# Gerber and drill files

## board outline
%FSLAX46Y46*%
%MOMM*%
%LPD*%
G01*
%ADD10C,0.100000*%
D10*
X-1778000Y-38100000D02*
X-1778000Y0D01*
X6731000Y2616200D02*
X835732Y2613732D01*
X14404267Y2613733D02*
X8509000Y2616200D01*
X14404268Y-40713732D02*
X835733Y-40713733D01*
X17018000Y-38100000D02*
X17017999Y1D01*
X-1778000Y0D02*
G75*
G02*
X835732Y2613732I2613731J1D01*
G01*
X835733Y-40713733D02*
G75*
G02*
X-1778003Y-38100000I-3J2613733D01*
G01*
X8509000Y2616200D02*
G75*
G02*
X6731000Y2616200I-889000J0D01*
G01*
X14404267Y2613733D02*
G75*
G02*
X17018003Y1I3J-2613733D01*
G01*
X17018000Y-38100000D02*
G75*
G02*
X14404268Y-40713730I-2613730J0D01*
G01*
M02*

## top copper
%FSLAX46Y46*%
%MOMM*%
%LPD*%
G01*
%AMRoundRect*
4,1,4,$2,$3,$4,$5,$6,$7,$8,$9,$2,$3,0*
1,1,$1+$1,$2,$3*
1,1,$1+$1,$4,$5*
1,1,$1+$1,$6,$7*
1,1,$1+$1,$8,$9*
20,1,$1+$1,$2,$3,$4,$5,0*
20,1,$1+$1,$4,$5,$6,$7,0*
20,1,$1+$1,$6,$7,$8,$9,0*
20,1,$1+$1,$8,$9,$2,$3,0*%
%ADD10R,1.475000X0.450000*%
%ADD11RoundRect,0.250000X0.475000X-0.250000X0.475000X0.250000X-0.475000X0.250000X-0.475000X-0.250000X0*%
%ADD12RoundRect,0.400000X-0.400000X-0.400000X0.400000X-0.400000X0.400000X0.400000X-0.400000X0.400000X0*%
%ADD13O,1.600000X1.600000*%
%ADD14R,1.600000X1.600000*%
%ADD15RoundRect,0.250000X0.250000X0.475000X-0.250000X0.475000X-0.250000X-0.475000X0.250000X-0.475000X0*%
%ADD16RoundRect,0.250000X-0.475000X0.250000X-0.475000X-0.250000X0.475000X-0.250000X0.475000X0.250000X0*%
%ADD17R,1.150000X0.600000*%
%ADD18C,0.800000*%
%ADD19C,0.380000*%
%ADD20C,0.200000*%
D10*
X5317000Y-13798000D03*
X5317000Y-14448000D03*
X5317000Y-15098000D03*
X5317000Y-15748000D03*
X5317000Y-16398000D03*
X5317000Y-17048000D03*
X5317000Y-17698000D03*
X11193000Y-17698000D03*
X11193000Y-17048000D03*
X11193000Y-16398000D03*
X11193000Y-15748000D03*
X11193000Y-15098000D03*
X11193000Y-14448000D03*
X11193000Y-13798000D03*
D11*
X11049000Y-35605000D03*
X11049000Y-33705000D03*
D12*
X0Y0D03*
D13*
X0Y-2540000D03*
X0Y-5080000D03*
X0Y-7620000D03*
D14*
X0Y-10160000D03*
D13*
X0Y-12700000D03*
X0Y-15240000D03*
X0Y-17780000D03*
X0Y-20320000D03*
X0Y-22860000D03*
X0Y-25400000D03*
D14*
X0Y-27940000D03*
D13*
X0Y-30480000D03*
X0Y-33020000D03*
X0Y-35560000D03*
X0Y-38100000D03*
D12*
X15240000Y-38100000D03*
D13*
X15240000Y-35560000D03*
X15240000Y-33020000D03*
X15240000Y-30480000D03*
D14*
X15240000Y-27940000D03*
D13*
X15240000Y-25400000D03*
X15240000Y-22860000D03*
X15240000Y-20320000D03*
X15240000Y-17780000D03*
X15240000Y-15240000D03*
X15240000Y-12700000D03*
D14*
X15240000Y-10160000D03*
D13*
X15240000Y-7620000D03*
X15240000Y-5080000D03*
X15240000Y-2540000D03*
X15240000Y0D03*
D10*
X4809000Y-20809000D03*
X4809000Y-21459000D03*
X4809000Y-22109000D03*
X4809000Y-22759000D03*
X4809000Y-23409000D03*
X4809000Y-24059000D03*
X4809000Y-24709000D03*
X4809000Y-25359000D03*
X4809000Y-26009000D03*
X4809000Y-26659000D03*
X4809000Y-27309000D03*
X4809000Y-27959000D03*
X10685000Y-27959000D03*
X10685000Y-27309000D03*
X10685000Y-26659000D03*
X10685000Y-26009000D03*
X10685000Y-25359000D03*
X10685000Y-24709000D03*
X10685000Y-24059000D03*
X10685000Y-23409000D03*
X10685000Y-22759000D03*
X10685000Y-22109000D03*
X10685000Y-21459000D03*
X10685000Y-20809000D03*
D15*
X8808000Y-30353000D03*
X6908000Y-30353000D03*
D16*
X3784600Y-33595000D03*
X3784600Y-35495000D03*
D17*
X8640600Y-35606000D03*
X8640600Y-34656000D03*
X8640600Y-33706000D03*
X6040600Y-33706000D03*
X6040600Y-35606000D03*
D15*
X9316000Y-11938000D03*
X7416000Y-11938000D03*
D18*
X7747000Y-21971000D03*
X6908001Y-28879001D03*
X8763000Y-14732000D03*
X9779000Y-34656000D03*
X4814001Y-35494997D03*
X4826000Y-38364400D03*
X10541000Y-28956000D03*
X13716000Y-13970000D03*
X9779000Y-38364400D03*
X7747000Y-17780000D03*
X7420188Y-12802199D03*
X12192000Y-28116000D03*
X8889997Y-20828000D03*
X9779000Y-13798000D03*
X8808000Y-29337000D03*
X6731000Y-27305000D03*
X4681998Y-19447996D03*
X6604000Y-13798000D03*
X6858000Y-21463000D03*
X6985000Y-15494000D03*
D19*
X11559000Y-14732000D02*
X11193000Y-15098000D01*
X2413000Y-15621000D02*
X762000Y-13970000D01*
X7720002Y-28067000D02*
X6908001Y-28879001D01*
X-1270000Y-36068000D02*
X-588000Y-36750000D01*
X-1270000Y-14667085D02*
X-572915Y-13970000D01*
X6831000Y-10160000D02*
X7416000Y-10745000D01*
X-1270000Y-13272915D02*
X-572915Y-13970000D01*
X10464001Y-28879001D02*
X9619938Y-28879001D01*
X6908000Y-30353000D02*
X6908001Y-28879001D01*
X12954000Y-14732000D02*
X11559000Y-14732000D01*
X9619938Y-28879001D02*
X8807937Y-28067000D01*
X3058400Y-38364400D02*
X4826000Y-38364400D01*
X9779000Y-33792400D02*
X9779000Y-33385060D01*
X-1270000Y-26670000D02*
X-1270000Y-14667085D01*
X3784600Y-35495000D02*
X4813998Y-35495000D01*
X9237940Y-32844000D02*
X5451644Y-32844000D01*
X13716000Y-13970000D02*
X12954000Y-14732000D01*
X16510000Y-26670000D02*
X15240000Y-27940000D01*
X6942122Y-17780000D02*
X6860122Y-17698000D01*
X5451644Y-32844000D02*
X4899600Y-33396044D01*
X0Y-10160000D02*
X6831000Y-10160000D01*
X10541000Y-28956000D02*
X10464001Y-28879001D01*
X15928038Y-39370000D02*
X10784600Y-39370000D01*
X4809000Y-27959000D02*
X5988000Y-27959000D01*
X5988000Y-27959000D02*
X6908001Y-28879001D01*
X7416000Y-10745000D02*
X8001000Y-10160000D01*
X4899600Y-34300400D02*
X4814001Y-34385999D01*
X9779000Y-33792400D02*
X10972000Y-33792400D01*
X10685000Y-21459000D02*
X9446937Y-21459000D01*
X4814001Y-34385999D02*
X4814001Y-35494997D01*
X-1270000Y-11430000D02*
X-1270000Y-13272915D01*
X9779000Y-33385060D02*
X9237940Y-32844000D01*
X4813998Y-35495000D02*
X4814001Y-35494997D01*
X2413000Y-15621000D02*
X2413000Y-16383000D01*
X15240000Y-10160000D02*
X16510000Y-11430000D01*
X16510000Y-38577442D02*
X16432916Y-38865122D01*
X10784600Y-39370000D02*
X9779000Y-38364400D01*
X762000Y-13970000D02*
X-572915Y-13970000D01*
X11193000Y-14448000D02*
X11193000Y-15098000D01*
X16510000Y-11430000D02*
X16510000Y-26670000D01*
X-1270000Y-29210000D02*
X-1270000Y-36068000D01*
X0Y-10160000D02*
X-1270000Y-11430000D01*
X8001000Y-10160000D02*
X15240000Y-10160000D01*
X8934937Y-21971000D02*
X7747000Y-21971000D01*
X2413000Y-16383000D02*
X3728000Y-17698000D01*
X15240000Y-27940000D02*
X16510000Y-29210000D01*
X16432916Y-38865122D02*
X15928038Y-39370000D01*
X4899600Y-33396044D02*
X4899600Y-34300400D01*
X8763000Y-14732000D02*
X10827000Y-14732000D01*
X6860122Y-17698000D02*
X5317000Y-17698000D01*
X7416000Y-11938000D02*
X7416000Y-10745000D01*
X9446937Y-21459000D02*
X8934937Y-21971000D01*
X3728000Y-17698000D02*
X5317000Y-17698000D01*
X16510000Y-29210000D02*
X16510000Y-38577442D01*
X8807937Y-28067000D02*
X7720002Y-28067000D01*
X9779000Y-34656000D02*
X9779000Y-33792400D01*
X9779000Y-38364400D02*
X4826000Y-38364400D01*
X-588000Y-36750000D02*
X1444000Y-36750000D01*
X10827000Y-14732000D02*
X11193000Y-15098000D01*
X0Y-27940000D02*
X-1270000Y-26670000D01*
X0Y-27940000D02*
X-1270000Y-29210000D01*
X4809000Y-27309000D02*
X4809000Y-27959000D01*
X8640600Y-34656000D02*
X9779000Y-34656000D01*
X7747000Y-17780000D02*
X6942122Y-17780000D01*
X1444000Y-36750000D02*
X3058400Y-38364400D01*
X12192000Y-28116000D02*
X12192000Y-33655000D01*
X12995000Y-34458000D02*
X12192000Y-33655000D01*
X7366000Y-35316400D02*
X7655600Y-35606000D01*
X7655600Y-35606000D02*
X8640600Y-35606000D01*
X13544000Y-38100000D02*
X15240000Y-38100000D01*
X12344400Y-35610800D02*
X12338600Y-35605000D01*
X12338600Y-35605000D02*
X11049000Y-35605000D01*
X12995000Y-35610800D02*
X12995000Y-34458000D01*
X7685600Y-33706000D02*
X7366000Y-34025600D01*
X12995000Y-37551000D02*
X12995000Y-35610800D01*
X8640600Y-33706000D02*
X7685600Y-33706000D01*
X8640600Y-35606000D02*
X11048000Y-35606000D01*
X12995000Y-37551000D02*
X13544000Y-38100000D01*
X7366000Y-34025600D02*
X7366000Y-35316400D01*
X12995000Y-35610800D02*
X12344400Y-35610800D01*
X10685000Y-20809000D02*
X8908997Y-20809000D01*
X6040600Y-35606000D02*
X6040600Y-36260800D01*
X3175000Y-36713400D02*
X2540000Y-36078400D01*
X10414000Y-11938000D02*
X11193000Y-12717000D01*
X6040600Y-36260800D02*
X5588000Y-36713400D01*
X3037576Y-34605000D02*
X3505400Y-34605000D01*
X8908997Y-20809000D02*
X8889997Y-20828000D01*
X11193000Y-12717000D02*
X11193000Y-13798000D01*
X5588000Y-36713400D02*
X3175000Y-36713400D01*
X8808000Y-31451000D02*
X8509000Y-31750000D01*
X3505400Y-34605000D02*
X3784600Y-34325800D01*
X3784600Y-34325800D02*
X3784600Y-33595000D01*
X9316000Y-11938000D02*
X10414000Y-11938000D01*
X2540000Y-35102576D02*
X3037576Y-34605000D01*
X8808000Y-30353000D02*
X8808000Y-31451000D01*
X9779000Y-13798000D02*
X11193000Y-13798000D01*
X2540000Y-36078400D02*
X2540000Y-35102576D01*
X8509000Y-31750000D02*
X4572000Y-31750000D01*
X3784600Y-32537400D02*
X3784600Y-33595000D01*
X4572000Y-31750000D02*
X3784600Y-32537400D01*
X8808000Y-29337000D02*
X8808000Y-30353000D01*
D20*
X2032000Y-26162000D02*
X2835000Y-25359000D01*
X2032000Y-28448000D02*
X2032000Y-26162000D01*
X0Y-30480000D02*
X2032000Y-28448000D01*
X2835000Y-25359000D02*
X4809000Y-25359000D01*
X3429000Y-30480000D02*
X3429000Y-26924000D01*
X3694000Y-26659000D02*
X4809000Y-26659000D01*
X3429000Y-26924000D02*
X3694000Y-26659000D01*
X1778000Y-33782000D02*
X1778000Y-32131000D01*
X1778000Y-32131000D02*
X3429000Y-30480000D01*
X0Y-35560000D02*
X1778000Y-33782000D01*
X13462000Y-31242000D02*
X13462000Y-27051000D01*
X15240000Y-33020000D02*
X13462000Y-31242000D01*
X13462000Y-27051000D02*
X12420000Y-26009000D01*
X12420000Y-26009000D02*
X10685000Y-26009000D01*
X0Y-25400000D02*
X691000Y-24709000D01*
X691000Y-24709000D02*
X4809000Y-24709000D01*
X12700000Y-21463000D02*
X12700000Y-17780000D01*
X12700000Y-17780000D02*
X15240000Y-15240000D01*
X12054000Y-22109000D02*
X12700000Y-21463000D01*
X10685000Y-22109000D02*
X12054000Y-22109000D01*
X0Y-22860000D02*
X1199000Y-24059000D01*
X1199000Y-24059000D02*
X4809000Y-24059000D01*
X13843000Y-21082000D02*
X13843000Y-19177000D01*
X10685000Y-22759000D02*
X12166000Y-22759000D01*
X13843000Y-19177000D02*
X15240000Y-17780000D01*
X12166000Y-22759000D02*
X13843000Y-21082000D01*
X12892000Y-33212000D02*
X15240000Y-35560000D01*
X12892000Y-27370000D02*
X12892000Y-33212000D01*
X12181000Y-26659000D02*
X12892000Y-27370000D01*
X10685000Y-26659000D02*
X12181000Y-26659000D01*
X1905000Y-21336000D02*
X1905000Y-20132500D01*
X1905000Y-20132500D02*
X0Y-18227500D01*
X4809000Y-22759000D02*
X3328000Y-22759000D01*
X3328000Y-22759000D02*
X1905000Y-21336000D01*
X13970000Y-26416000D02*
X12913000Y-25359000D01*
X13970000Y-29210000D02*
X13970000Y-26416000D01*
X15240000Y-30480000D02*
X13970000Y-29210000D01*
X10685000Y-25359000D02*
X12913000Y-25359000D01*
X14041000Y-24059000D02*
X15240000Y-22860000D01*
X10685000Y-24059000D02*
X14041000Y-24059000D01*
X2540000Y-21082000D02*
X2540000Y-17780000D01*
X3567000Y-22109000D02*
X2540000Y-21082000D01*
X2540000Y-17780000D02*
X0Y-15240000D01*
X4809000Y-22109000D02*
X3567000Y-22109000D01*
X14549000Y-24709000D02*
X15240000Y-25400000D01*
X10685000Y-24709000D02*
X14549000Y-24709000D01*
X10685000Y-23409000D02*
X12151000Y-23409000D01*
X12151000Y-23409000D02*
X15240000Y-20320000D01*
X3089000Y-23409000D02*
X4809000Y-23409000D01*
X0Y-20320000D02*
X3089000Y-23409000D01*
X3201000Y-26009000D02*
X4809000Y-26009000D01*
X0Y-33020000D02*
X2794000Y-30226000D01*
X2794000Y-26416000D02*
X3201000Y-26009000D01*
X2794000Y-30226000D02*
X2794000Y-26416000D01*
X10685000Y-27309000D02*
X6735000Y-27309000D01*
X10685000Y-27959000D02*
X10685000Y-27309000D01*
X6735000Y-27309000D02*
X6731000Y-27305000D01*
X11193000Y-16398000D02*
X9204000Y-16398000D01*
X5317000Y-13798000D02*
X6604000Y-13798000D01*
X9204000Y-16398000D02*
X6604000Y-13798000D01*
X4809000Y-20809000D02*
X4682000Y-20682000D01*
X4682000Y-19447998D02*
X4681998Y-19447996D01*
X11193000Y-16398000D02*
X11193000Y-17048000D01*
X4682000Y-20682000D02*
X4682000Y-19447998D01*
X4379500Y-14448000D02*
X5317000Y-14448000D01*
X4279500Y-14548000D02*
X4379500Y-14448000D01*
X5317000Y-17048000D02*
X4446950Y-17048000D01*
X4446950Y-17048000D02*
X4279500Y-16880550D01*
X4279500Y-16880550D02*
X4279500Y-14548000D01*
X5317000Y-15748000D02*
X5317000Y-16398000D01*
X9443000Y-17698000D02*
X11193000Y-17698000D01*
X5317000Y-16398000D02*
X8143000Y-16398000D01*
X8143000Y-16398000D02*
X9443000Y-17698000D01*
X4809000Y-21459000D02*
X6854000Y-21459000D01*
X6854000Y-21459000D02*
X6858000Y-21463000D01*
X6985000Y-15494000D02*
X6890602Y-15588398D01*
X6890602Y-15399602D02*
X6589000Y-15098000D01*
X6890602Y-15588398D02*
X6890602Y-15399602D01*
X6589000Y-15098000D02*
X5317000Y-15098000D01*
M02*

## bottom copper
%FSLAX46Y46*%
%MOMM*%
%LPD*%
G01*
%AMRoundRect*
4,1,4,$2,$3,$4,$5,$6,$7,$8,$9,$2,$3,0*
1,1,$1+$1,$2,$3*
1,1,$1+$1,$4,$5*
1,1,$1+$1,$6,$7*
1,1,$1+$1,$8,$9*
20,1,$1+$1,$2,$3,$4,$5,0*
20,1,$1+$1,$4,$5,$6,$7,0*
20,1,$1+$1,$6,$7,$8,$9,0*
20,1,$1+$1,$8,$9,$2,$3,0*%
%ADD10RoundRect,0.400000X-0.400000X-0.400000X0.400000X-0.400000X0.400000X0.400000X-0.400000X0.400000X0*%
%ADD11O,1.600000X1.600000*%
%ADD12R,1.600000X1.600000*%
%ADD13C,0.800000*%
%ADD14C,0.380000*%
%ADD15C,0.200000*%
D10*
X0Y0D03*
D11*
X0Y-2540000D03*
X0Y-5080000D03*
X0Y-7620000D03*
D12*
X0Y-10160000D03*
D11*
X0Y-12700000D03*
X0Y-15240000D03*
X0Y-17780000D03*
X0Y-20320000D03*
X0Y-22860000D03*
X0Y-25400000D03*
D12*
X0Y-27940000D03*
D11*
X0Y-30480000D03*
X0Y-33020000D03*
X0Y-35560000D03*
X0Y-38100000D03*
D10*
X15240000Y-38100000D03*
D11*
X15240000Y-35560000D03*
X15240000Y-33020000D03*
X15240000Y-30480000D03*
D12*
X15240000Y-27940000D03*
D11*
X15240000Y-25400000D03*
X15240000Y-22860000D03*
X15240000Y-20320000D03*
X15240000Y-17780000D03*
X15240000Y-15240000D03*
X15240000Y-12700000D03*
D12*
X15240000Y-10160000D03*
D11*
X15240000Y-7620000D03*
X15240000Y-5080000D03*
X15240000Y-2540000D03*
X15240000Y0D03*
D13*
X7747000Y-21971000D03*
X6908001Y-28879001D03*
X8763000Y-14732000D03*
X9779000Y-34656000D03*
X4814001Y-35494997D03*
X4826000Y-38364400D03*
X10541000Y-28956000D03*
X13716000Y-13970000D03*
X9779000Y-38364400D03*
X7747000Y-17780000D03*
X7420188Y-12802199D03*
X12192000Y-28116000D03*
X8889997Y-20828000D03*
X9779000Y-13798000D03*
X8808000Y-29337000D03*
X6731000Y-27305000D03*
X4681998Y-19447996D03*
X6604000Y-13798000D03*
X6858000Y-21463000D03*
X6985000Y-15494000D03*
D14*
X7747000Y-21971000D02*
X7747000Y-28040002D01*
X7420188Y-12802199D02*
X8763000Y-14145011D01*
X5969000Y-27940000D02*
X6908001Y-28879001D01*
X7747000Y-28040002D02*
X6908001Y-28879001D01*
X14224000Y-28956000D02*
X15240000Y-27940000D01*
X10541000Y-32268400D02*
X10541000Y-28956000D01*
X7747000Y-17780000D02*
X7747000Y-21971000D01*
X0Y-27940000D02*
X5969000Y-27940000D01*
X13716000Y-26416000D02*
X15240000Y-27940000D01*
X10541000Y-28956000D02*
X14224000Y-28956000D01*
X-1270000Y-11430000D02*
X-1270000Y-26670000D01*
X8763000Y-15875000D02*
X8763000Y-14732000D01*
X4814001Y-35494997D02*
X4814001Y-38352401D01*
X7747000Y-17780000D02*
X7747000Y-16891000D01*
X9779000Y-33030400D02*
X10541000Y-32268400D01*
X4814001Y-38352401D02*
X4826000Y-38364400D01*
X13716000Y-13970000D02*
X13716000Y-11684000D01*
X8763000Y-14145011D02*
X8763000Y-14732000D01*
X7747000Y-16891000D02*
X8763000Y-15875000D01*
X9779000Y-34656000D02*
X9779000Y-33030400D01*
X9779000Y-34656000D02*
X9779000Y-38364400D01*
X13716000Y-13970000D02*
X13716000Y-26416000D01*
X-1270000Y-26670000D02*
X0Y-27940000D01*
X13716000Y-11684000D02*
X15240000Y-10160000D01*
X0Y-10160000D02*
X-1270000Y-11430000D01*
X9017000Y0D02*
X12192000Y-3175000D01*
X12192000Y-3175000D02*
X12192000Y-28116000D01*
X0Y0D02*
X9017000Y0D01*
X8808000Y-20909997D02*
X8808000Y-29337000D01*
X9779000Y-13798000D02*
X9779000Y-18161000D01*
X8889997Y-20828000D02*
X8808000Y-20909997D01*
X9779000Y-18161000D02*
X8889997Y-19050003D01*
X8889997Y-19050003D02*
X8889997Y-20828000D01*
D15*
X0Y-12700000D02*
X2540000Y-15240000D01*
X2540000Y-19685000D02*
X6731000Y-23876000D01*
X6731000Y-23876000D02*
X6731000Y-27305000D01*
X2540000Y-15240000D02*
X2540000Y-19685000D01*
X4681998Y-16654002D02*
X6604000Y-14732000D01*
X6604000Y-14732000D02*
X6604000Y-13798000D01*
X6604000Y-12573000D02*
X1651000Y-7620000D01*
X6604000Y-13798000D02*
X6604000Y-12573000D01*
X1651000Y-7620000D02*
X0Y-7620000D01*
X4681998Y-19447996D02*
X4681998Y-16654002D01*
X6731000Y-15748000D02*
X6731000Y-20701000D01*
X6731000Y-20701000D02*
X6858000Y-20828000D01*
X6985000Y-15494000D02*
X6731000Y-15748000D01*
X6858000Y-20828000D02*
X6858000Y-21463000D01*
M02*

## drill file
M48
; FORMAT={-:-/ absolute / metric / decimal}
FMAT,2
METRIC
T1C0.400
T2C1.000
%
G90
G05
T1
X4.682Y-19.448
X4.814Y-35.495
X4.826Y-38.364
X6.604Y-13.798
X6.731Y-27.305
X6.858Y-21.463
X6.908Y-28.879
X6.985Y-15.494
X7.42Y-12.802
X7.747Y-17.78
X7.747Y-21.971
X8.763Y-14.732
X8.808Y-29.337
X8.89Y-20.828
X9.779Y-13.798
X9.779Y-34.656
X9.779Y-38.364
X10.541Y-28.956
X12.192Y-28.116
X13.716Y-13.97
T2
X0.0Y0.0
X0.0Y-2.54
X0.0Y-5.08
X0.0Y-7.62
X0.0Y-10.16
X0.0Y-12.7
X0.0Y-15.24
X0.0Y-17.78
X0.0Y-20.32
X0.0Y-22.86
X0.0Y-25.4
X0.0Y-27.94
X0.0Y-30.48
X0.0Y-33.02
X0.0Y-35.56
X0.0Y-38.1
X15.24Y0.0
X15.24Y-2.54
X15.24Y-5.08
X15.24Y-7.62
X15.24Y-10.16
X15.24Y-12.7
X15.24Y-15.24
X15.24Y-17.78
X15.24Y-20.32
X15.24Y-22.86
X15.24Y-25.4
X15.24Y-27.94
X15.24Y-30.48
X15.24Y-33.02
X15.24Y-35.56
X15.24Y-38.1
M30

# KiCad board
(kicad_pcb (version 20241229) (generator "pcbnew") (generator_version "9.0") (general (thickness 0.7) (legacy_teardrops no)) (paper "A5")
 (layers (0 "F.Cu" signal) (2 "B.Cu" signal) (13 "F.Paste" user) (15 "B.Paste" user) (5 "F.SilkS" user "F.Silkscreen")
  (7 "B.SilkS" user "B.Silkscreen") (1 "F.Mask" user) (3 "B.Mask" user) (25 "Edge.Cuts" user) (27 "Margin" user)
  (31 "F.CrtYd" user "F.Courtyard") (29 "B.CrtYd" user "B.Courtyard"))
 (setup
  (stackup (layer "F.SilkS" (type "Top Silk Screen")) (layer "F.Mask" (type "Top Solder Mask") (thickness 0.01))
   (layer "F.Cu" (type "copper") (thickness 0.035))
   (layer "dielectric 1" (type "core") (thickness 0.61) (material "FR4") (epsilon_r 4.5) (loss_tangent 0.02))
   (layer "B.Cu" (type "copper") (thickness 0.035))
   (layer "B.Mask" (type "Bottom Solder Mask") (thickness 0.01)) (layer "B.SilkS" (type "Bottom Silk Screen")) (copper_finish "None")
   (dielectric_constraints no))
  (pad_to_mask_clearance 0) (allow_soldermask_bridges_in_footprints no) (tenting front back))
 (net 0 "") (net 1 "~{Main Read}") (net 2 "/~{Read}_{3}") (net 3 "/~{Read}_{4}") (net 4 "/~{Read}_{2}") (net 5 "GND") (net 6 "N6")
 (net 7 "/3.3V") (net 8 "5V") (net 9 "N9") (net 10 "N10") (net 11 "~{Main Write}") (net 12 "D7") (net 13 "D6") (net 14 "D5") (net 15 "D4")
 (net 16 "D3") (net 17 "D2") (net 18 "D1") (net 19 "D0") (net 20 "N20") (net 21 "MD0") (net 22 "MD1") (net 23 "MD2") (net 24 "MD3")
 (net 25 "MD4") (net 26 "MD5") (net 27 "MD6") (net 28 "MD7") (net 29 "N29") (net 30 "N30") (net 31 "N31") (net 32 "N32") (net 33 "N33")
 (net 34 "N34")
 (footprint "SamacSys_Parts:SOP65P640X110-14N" (layer "F.Cu") (at 8.255 15.748)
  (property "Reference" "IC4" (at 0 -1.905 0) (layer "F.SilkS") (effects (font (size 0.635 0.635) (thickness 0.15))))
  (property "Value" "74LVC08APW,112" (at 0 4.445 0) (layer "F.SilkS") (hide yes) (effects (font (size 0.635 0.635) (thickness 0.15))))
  (pad "1" smd rect (at -2.938 -1.95 90) (size 0.45 1.475) (layers "F.Cu" "F.Mask" "F.Paste") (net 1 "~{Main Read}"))
  (pad "2" smd rect (at -2.938 -1.3 90) (size 0.45 1.475) (layers "F.Cu" "F.Mask" "F.Paste") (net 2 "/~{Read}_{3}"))
  (pad "3" smd rect (at -2.938 -0.65 90) (size 0.45 1.475) (layers "F.Cu" "F.Mask" "F.Paste") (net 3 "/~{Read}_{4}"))
  (pad "4" smd rect (at -2.938 0 90) (size 0.45 1.475) (layers "F.Cu" "F.Mask" "F.Paste") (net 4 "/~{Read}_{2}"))
  (pad "5" smd rect (at -2.938 0.65 90) (size 0.45 1.475) (layers "F.Cu" "F.Mask" "F.Paste") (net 4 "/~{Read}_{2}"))
  (pad "6" smd rect (at -2.938 1.3 90) (size 0.45 1.475) (layers "F.Cu" "F.Mask" "F.Paste") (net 2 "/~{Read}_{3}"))
  (pad "7" smd rect (at -2.938 1.95 90) (size 0.45 1.475) (layers "F.Cu" "F.Mask" "F.Paste") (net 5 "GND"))
  (pad "8" smd rect (at 2.938 1.95 90) (size 0.45 1.475) (layers "F.Cu" "F.Mask" "F.Paste") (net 4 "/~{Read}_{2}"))
  (pad "9" smd rect (at 2.938 1.3 90) (size 0.45 1.475) (layers "F.Cu" "F.Mask" "F.Paste") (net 1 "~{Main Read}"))
  (pad "10" smd rect (at 2.938 0.65 90) (size 0.45 1.475) (layers "F.Cu" "F.Mask" "F.Paste") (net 1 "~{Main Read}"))
  (pad "11" smd rect (at 2.938 0 90) (size 0.45 1.475) (layers "F.Cu" "F.Mask" "F.Paste") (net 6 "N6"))
  (pad "12" smd rect (at 2.938 -0.65 90) (size 0.45 1.475) (layers "F.Cu" "F.Mask" "F.Paste") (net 5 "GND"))
  (pad "13" smd rect (at 2.938 -1.3 90) (size 0.45 1.475) (layers "F.Cu" "F.Mask" "F.Paste") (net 5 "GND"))
  (pad "14" smd rect (at 2.938 -1.95 90) (size 0.45 1.475) (layers "F.Cu" "F.Mask" "F.Paste") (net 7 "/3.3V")))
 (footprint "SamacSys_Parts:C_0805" (layer "F.Cu") (at 11.049 34.671)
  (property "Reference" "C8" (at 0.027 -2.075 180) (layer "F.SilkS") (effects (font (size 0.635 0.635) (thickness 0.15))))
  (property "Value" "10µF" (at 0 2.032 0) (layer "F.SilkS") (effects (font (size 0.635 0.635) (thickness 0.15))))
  (pad "1" smd roundrect (at 0 0.934 90) (size 1 1.45) (layers "F.Cu" "F.Mask" "F.Paste") (roundrect_rratio 0.25) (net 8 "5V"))
  (pad "2" smd roundrect (at 0 -0.966 90) (size 1 1.45) (layers "F.Cu" "F.Mask" "F.Paste") (roundrect_rratio 0.25) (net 5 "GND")))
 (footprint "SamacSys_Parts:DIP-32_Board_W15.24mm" (layer "F.Cu") (at 0 0)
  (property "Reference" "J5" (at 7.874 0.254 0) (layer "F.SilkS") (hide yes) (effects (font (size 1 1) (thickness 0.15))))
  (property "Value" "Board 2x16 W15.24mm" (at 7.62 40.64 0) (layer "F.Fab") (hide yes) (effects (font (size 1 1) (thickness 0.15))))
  (fp_line (start -1.778 38.1) (end -1.778 0) (stroke (width 0.1) (type solid)) (layer "Edge.Cuts"))
  (fp_line (start 6.731 -2.6162) (end 0.835732 -2.613732) (stroke (width 0.1) (type solid)) (layer "Edge.Cuts"))
  (fp_line (start 14.404267 -2.613733) (end 8.509 -2.6162) (stroke (width 0.1) (type solid)) (layer "Edge.Cuts"))
  (fp_line (start 14.404268 40.713732) (end 0.835733 40.713733) (stroke (width 0.1) (type solid)) (layer "Edge.Cuts"))
  (fp_line (start 17.018 38.1) (end 17.017999 -0.000001) (stroke (width 0.1) (type solid)) (layer "Edge.Cuts"))
  (fp_arc (start -1.778 0) (mid -1.012456 -1.848188) (end 0.835732 -2.613732) (stroke (width 0.1) (type solid)) (layer "Edge.Cuts"))
  (fp_arc (start 0.835733 40.713733) (mid -1.012456 39.948189) (end -1.778 38.1) (stroke (width 0.1) (type solid)) (layer "Edge.Cuts"))
  (fp_arc (start 8.509 -2.6162) (mid 7.62 -1.7272) (end 6.731 -2.6162) (stroke (width 0.1) (type default)) (layer "Edge.Cuts"))
  (fp_arc (start 14.404267 -2.613733) (mid 16.252455 -1.848189) (end 17.017999 -0.000001) (stroke (width 0.1) (type solid))
   (layer "Edge.Cuts"))
  (fp_arc (start 17.018 38.1) (mid 16.252455 39.948187) (end 14.404268 40.713732) (stroke (width 0.1) (type solid)) (layer "Edge.Cuts"))
  (pad "1" thru_hole roundrect (at 0 0) (size 1.6 1.6) (drill 1) (layers "*.Cu" "*.Mask") (remove_unused_layers no) (roundrect_rratio 0.25)
   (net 8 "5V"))
  (pad "2" thru_hole oval (at 0 2.54) (size 1.6 1.6) (drill 1) (layers "*.Cu" "*.Mask") (remove_unused_layers no) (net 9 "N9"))
  (pad "3" thru_hole oval (at 0 5.08) (size 1.6 1.6) (drill 1) (layers "*.Cu" "*.Mask") (remove_unused_layers no) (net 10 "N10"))
  (pad "4" thru_hole oval (at 0 7.62) (size 1.6 1.6) (drill 1) (layers "*.Cu" "*.Mask") (remove_unused_layers no) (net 1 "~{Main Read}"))
  (pad "5" thru_hole rect (at 0 10.16) (size 1.6 1.6) (drill 1) (layers "*.Cu" "*.Mask") (remove_unused_layers no) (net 5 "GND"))
  (pad "6" thru_hole oval (at 0 12.7) (size 1.6 1.6) (drill 1) (layers "*.Cu" "*.Mask") (remove_unused_layers no) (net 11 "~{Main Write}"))
  (pad "7" thru_hole oval (at 0 15.24) (size 1.6 1.6) (drill 1) (layers "*.Cu" "*.Mask") (remove_unused_layers no) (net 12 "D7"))
  (pad "8" thru_hole oval (at 0 17.78) (size 1.6 1.6) (drill 1) (layers "*.Cu" "*.Mask") (remove_unused_layers no) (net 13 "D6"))
  (pad "9" thru_hole oval (at 0 20.32) (size 1.6 1.6) (drill 1) (layers "*.Cu" "*.Mask") (remove_unused_layers no) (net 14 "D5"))
  (pad "10" thru_hole oval (at 0 22.86) (size 1.6 1.6) (drill 1) (layers "*.Cu" "*.Mask") (remove_unused_layers no) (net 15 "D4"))
  (pad "11" thru_hole oval (at 0 25.4) (size 1.6 1.6) (drill 1) (layers "*.Cu" "*.Mask") (remove_unused_layers no) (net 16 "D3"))
  (pad "12" thru_hole rect (at 0 27.94) (size 1.6 1.6) (drill 1) (layers "*.Cu" "*.Mask") (remove_unused_layers no) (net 5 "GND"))
  (pad "13" thru_hole oval (at 0 30.48) (size 1.6 1.6) (drill 1) (layers "*.Cu" "*.Mask") (remove_unused_layers no) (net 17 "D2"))
  (pad "14" thru_hole oval (at 0 33.02) (size 1.6 1.6) (drill 1) (layers "*.Cu" "*.Mask") (remove_unused_layers no) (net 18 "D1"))
  (pad "15" thru_hole oval (at 0 35.56) (size 1.6 1.6) (drill 1) (layers "*.Cu" "*.Mask") (remove_unused_layers no) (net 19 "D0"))
  (pad "16" thru_hole oval (at 0 38.1) (size 1.6 1.6) (drill 1) (layers "*.Cu" "*.Mask") (remove_unused_layers no) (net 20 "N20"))
  (pad "17" thru_hole roundrect (at 15.24 38.1) (size 1.6 1.6) (drill 1) (layers "*.Cu" "*.Mask") (remove_unused_layers no)
   (roundrect_rratio 0.25) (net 8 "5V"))
  (pad "18" thru_hole oval (at 15.24 35.56 180) (size 1.6 1.6) (drill 1) (layers "*.Cu" "*.Mask") (remove_unused_layers no) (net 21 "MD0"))
  (pad "19" thru_hole oval (at 15.24 33.02 180) (size 1.6 1.6) (drill 1) (layers "*.Cu" "*.Mask") (remove_unused_layers no) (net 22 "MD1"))
  (pad "20" thru_hole oval (at 15.24 30.48 180) (size 1.6 1.6) (drill 1) (layers "*.Cu" "*.Mask") (remove_unused_layers no) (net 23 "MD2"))
  (pad "21" thru_hole rect (at 15.24 27.94) (size 1.6 1.6) (drill 1) (layers "*.Cu" "*.Mask") (remove_unused_layers no) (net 5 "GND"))
  (pad "22" thru_hole oval (at 15.24 25.4) (size 1.6 1.6) (drill 1) (layers "*.Cu" "*.Mask") (remove_unused_layers no) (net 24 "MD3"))
  (pad "23" thru_hole oval (at 15.24 22.86) (size 1.6 1.6) (drill 1) (layers "*.Cu" "*.Mask") (remove_unused_layers no) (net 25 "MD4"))
  (pad "24" thru_hole oval (at 15.24 20.32) (size 1.6 1.6) (drill 1) (layers "*.Cu" "*.Mask") (remove_unused_layers no) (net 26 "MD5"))
  (pad "25" thru_hole oval (at 15.24 17.78) (size 1.6 1.6) (drill 1) (layers "*.Cu" "*.Mask") (remove_unused_layers no) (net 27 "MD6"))
  (pad "26" thru_hole oval (at 15.24 15.24) (size 1.6 1.6) (drill 1) (layers "*.Cu" "*.Mask") (remove_unused_layers no) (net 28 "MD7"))
  (pad "27" thru_hole oval (at 15.24 12.7) (size 1.6 1.6) (drill 1) (layers "*.Cu" "*.Mask") (remove_unused_layers no) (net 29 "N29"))
  (pad "28" thru_hole rect (at 15.24 10.16) (size 1.6 1.6) (drill 1) (layers "*.Cu" "*.Mask") (remove_unused_layers no) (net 5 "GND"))
  (pad "29" thru_hole oval (at 15.24 7.62) (size 1.6 1.6) (drill 1) (layers "*.Cu" "*.Mask") (remove_unused_layers no) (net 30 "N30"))
  (pad "30" thru_hole oval (at 15.24 5.08) (size 1.6 1.6) (drill 1) (layers "*.Cu" "*.Mask") (remove_unused_layers no) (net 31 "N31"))
  (pad "31" thru_hole oval (at 15.24 2.54) (size 1.6 1.6) (drill 1) (layers "*.Cu" "*.Mask") (remove_unused_layers no) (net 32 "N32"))
  (pad "32" thru_hole oval (at 15.24 0) (size 1.6 1.6) (drill 1) (layers "*.Cu" "*.Mask") (remove_unused_layers no) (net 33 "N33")))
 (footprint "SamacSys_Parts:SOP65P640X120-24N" (layer "F.Cu") (at 7.747 24.384)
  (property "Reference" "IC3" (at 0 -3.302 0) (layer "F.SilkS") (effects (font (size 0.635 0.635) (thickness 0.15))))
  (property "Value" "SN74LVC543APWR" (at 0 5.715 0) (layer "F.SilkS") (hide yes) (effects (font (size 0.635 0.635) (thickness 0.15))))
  (pad "1" smd rect (at -2.938 -3.575 90) (size 0.45 1.475) (layers "F.Cu" "F.Mask" "F.Paste") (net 1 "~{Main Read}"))
  (pad "2" smd rect (at -2.938 -2.925 90) (size 0.45 1.475) (layers "F.Cu" "F.Mask" "F.Paste") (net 3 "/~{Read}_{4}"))
  (pad "3" smd rect (at -2.938 -2.275 90) (size 0.45 1.475) (layers "F.Cu" "F.Mask" "F.Paste") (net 12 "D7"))
  (pad "4" smd rect (at -2.938 -1.625 90) (size 0.45 1.475) (layers "F.Cu" "F.Mask" "F.Paste") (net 13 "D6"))
  (pad "5" smd rect (at -2.938 -0.975 90) (size 0.45 1.475) (layers "F.Cu" "F.Mask" "F.Paste") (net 14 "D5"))
  (pad "6" smd rect (at -2.938 -0.325 90) (size 0.45 1.475) (layers "F.Cu" "F.Mask" "F.Paste") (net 15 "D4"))
  (pad "7" smd rect (at -2.938 0.325 90) (size 0.45 1.475) (layers "F.Cu" "F.Mask" "F.Paste") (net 16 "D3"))
  (pad "8" smd rect (at -2.938 0.975 90) (size 0.45 1.475) (layers "F.Cu" "F.Mask" "F.Paste") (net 17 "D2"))
  (pad "9" smd rect (at -2.938 1.625 90) (size 0.45 1.475) (layers "F.Cu" "F.Mask" "F.Paste") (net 18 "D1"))
  (pad "10" smd rect (at -2.938 2.275 90) (size 0.45 1.475) (layers "F.Cu" "F.Mask" "F.Paste") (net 19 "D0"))
  (pad "11" smd rect (at -2.938 2.925 90) (size 0.45 1.475) (layers "F.Cu" "F.Mask" "F.Paste") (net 5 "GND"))
  (pad "12" smd rect (at -2.938 3.575 90) (size 0.45 1.475) (layers "F.Cu" "F.Mask" "F.Paste") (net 5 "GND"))
  (pad "13" smd rect (at 2.938 3.575 90) (size 0.45 1.475) (layers "F.Cu" "F.Mask" "F.Paste") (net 11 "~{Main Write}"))
  (pad "14" smd rect (at 2.938 2.925 90) (size 0.45 1.475) (layers "F.Cu" "F.Mask" "F.Paste") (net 11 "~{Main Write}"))
  (pad "15" smd rect (at 2.938 2.275 90) (size 0.45 1.475) (layers "F.Cu" "F.Mask" "F.Paste") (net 21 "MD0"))
  (pad "16" smd rect (at 2.938 1.625 90) (size 0.45 1.475) (layers "F.Cu" "F.Mask" "F.Paste") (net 22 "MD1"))
  (pad "17" smd rect (at 2.938 0.975 90) (size 0.45 1.475) (layers "F.Cu" "F.Mask" "F.Paste") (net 23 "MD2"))
  (pad "18" smd rect (at 2.938 0.325 90) (size 0.45 1.475) (layers "F.Cu" "F.Mask" "F.Paste") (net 24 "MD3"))
  (pad "19" smd rect (at 2.938 -0.325 90) (size 0.45 1.475) (layers "F.Cu" "F.Mask" "F.Paste") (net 25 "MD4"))
  (pad "20" smd rect (at 2.938 -0.975 90) (size 0.45 1.475) (layers "F.Cu" "F.Mask" "F.Paste") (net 26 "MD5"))
  (pad "21" smd rect (at 2.938 -1.625 90) (size 0.45 1.475) (layers "F.Cu" "F.Mask" "F.Paste") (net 27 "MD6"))
  (pad "22" smd rect (at 2.938 -2.275 90) (size 0.45 1.475) (layers "F.Cu" "F.Mask" "F.Paste") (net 28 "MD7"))
  (pad "23" smd rect (at 2.938 -2.925 90) (size 0.45 1.475) (layers "F.Cu" "F.Mask" "F.Paste") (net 5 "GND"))
  (pad "24" smd rect (at 2.938 -3.575 90) (size 0.45 1.475) (layers "F.Cu" "F.Mask" "F.Paste") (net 7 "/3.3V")))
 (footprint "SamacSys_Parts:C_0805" (layer "F.Cu") (at 7.874 30.353 90)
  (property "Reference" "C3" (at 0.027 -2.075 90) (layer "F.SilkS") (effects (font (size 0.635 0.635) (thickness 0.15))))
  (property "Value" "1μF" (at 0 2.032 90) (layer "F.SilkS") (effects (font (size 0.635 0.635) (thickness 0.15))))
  (pad "1" smd roundrect (at 0 0.934 180) (size 1 1.45) (layers "F.Cu" "F.Mask" "F.Paste") (roundrect_rratio 0.25) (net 7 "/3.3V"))
  (pad "2" smd roundrect (at 0 -0.966 180) (size 1 1.45) (layers "F.Cu" "F.Mask" "F.Paste") (roundrect_rratio 0.25) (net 5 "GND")))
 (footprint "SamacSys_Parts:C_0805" (layer "F.Cu") (at 3.7846 34.529 180)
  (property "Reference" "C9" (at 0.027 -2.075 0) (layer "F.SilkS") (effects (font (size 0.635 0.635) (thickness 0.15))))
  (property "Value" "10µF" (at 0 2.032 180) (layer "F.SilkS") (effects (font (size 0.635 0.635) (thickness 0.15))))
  (pad "1" smd roundrect (at 0 0.934 270) (size 1 1.45) (layers "F.Cu" "F.Mask" "F.Paste") (roundrect_rratio 0.25) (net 7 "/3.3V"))
  (pad "2" smd roundrect (at 0 -0.966 270) (size 1 1.45) (layers "F.Cu" "F.Mask" "F.Paste") (roundrect_rratio 0.25) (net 5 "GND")))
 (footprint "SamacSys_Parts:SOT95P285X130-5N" (layer "F.Cu") (at 7.3406 34.656 180)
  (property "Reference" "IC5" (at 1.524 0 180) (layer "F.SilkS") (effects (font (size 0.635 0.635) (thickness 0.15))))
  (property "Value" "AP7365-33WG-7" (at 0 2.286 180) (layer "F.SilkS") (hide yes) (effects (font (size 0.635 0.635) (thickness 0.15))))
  (pad "1" smd rect (at -1.3 -0.95 270) (size 0.6 1.15) (layers "F.Cu" "F.Mask" "F.Paste") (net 8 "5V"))
  (pad "2" smd rect (at -1.3 0 270) (size 0.6 1.15) (layers "F.Cu" "F.Mask" "F.Paste") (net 5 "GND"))
  (pad "3" smd rect (at -1.3 0.95 270) (size 0.6 1.15) (layers "F.Cu" "F.Mask" "F.Paste") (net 8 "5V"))
  (pad "4" smd rect (at 1.3 0.95 270) (size 0.6 1.15) (layers "F.Cu" "F.Mask" "F.Paste") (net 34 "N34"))
  (pad "5" smd rect (at 1.3 -0.95 270) (size 0.6 1.15) (layers "F.Cu" "F.Mask" "F.Paste") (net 7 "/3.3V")))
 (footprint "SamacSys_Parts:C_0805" (layer "F.Cu") (at 8.382 11.938 90)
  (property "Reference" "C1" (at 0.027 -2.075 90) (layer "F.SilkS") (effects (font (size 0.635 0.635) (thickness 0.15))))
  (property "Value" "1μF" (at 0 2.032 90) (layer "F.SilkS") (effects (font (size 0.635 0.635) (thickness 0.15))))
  (pad "1" smd roundrect (at 0 0.934 180) (size 1 1.45) (layers "F.Cu" "F.Mask" "F.Paste") (roundrect_rratio 0.25) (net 7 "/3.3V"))
  (pad "2" smd roundrect (at 0 -0.966 180) (size 1 1.45) (layers "F.Cu" "F.Mask" "F.Paste") (roundrect_rratio 0.25) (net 5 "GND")))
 (segment (start 11.559 14.732) (end 11.193 15.098) (width 0.38) (layer "F.Cu") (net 5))
 (segment (start 2.413 15.621) (end 0.762 13.97) (width 0.38) (layer "F.Cu") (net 5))
 (segment (start 7.720002 28.067) (end 6.908001 28.879001) (width 0.38) (layer "F.Cu") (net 5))
 (segment (start -1.27 36.068) (end -0.588 36.75) (width 0.38) (layer "F.Cu") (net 5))
 (segment (start -1.27 14.667085) (end -0.572915 13.97) (width 0.38) (layer "F.Cu") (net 5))
 (segment (start 6.831 10.16) (end 7.416 10.745) (width 0.38) (layer "F.Cu") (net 5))
 (segment (start -1.27 13.272915) (end -0.572915 13.97) (width 0.38) (layer "F.Cu") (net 5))
 (segment (start 10.464001 28.879001) (end 9.619938 28.879001) (width 0.38) (layer "F.Cu") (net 5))
 (segment (start 6.908 30.353) (end 6.908001 28.879001) (width 0.38) (layer "F.Cu") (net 5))
 (segment (start 12.954 14.732) (end 11.559 14.732) (width 0.38) (layer "F.Cu") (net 5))
 (segment (start 9.619938 28.879001) (end 8.807937 28.067) (width 0.38) (layer "F.Cu") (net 5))
 (segment (start 3.0584 38.3644) (end 4.826 38.3644) (width 0.38) (layer "F.Cu") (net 5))
 (segment (start 9.779 33.7924) (end 9.779 33.38506) (width 0.38) (layer "F.Cu") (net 5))
 (segment (start -1.27 26.67) (end -1.27 14.667085) (width 0.38) (layer "F.Cu") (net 5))
 (segment (start 3.7846 35.495) (end 4.813998 35.495) (width 0.38) (layer "F.Cu") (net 5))
 (segment (start 9.23794 32.844) (end 5.451644 32.844) (width 0.38) (layer "F.Cu") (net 5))
 (segment (start 13.716 13.97) (end 12.954 14.732) (width 0.38) (layer "F.Cu") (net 5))
 (segment (start 16.51 26.67) (end 15.24 27.94) (width 0.38) (layer "F.Cu") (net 5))
 (segment (start 6.942122 17.78) (end 6.860122 17.698) (width 0.38) (layer "F.Cu") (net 5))
 (segment (start 5.451644 32.844) (end 4.8996 33.396044) (width 0.38) (layer "F.Cu") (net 5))
 (segment (start 0 10.16) (end 6.831 10.16) (width 0.38) (layer "F.Cu") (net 5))
 (segment (start 10.541 28.956) (end 10.464001 28.879001) (width 0.38) (layer "F.Cu") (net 5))
 (segment (start 15.928038 39.37) (end 10.7846 39.37) (width 0.38) (layer "F.Cu") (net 5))
 (segment (start 4.809 27.959) (end 5.988 27.959) (width 0.38) (layer "F.Cu") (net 5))
 (segment (start 5.988 27.959) (end 6.908001 28.879001) (width 0.38) (layer "F.Cu") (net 5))
 (segment (start 7.416 10.745) (end 8.001 10.16) (width 0.38) (layer "F.Cu") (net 5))
 (segment (start 4.8996 34.3004) (end 4.814001 34.385999) (width 0.38) (layer "F.Cu") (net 5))
 (segment (start 9.779 33.7924) (end 10.972 33.7924) (width 0.38) (layer "F.Cu") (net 5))
 (segment (start 10.685 21.459) (end 9.446937 21.459) (width 0.38) (layer "F.Cu") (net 5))
 (segment (start 4.814001 34.385999) (end 4.814001 35.494997) (width 0.38) (layer "F.Cu") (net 5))
 (segment (start -1.27 11.43) (end -1.27 13.272915) (width 0.38) (layer "F.Cu") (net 5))
 (segment (start 9.779 33.38506) (end 9.23794 32.844) (width 0.38) (layer "F.Cu") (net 5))
 (segment (start 4.813998 35.495) (end 4.814001 35.494997) (width 0.38) (layer "F.Cu") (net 5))
 (segment (start 2.413 15.621) (end 2.413 16.383) (width 0.38) (layer "F.Cu") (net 5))
 (segment (start 15.24 10.16) (end 16.51 11.43) (width 0.38) (layer "F.Cu") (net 5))
 (segment (start 16.51 38.577442) (end 16.432916 38.865122) (width 0.38) (layer "F.Cu") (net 5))
 (segment (start 10.7846 39.37) (end 9.779 38.3644) (width 0.38) (layer "F.Cu") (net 5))
 (segment (start 0.762 13.97) (end -0.572915 13.97) (width 0.38) (layer "F.Cu") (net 5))
 (segment (start 11.193 14.448) (end 11.193 15.098) (width 0.38) (layer "F.Cu") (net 5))
 (segment (start 16.51 11.43) (end 16.51 26.67) (width 0.38) (layer "F.Cu") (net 5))
 (segment (start -1.27 29.21) (end -1.27 36.068) (width 0.38) (layer "F.Cu") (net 5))
 (segment (start 0 10.16) (end -1.27 11.43) (width 0.38) (layer "F.Cu") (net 5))
 (segment (start 8.001 10.16) (end 15.24 10.16) (width 0.38) (layer "F.Cu") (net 5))
 (segment (start 8.934937 21.971) (end 7.747 21.971) (width 0.38) (layer "F.Cu") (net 5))
 (segment (start 2.413 16.383) (end 3.728 17.698) (width 0.38) (layer "F.Cu") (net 5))
 (segment (start 15.24 27.94) (end 16.51 29.21) (width 0.38) (layer "F.Cu") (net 5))
 (segment (start 16.432916 38.865122) (end 15.928038 39.37) (width 0.38) (layer "F.Cu") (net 5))
 (segment (start 4.8996 33.396044) (end 4.8996 34.3004) (width 0.38) (layer "F.Cu") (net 5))
 (segment (start 8.763 14.732) (end 10.827 14.732) (width 0.38) (layer "F.Cu") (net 5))
 (segment (start 6.860122 17.698) (end 5.317 17.698) (width 0.38) (layer "F.Cu") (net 5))
 (segment (start 7.416 11.938) (end 7.416 10.745) (width 0.38) (layer "F.Cu") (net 5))
 (segment (start 9.446937 21.459) (end 8.934937 21.971) (width 0.38) (layer "F.Cu") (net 5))
 (segment (start 3.728 17.698) (end 5.317 17.698) (width 0.38) (layer "F.Cu") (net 5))
 (segment (start 16.51 29.21) (end 16.51 38.577442) (width 0.38) (layer "F.Cu") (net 5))
 (segment (start 8.807937 28.067) (end 7.720002 28.067) (width 0.38) (layer "F.Cu") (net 5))
 (segment (start 9.779 34.656) (end 9.779 33.7924) (width 0.38) (layer "F.Cu") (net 5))
 (segment (start 9.779 38.3644) (end 4.826 38.3644) (width 0.38) (layer "F.Cu") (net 5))
 (segment (start -0.588 36.75) (end 1.444 36.75) (width 0.38) (layer "F.Cu") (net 5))
 (segment (start 10.827 14.732) (end 11.193 15.098) (width 0.38) (layer "F.Cu") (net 5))
 (segment (start 0 27.94) (end -1.27 26.67) (width 0.38) (layer "F.Cu") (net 5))
 (segment (start 0 27.94) (end -1.27 29.21) (width 0.38) (layer "F.Cu") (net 5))
 (segment (start 4.809 27.309) (end 4.809 27.959) (width 0.38) (layer "F.Cu") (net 5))
 (segment (start 8.6406 34.656) (end 9.779 34.656) (width 0.38) (layer "F.Cu") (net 5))
 (segment (start 7.747 17.78) (end 6.942122 17.78) (width 0.38) (layer "F.Cu") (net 5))
 (segment (start 1.444 36.75) (end 3.0584 38.3644) (width 0.38) (layer "F.Cu") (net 5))
 (via (at 7.747 21.971) (size 0.8) (drill 0.4) (layers "F.Cu" "B.Cu") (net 5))
 (via (at 6.908001 28.879001) (size 0.8) (drill 0.4) (layers "F.Cu" "B.Cu") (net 5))
 (via (at 8.763 14.732) (size 0.8) (drill 0.4) (layers "F.Cu" "B.Cu") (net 5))
 (via (at 9.779 34.656) (size 0.8) (drill 0.4) (layers "F.Cu" "B.Cu") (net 5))
 (via (at 4.814001 35.494997) (size 0.8) (drill 0.4) (layers "F.Cu" "B.Cu") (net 5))
 (via (at 4.826 38.3644) (size 0.8) (drill 0.4) (layers "F.Cu" "B.Cu") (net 5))
 (via (at 10.541 28.956) (size 0.8) (drill 0.4) (layers "F.Cu" "B.Cu") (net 5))
 (via (at 13.716 13.97) (size 0.8) (drill 0.4) (layers "F.Cu" "B.Cu") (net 5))
 (via (at 9.779 38.3644) (size 0.8) (drill 0.4) (layers "F.Cu" "B.Cu") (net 5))
 (via (at 7.747 17.78) (size 0.8) (drill 0.4) (layers "F.Cu" "B.Cu") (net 5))
 (via (at 7.420188 12.802199) (size 0.8) (drill 0.4) (layers "F.Cu" "B.Cu") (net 5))
 (segment (start 7.747 21.971) (end 7.747 28.040002) (width 0.38) (layer "B.Cu") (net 5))
 (segment (start 7.420188 12.802199) (end 8.763 14.145011) (width 0.38) (layer "B.Cu") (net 5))
 (segment (start 5.969 27.94) (end 6.908001 28.879001) (width 0.38) (layer "B.Cu") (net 5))
 (segment (start 7.747 28.040002) (end 6.908001 28.879001) (width 0.38) (layer "B.Cu") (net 5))
 (segment (start 14.224 28.956) (end 15.24 27.94) (width 0.38) (layer "B.Cu") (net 5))
 (segment (start 10.541 32.2684) (end 10.541 28.956) (width 0.38) (layer "B.Cu") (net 5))
 (segment (start 7.747 17.78) (end 7.747 21.971) (width 0.38) (layer "B.Cu") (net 5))
 (segment (start 0 27.94) (end 5.969 27.94) (width 0.38) (layer "B.Cu") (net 5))
 (segment (start 13.716 26.416) (end 15.24 27.94) (width 0.38) (layer "B.Cu") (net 5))
 (segment (start 10.541 28.956) (end 14.224 28.956) (width 0.38) (layer "B.Cu") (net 5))
 (segment (start -1.27 11.43) (end -1.27 26.67) (width 0.38) (layer "B.Cu") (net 5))
 (segment (start 8.763 15.875) (end 8.763 14.732) (width 0.38) (layer "B.Cu") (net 5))
 (segment (start 4.814001 35.494997) (end 4.814001 38.352401) (width 0.38) (layer "B.Cu") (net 5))
 (segment (start 7.747 17.78) (end 7.747 16.891) (width 0.38) (layer "B.Cu") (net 5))
 (segment (start 9.779 33.0304) (end 10.541 32.2684) (width 0.38) (layer "B.Cu") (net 5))
 (segment (start 4.814001 38.352401) (end 4.826 38.3644) (width 0.38) (layer "B.Cu") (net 5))
 (segment (start 13.716 13.97) (end 13.716 11.684) (width 0.38) (layer "B.Cu") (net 5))
 (segment (start 8.763 14.145011) (end 8.763 14.732) (width 0.38) (layer "B.Cu") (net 5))
 (segment (start 7.747 16.891) (end 8.763 15.875) (width 0.38) (layer "B.Cu") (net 5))
 (segment (start 9.779 34.656) (end 9.779 33.0304) (width 0.38) (layer "B.Cu") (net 5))
 (segment (start 9.779 34.656) (end 9.779 38.3644) (width 0.38) (layer "B.Cu") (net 5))
 (segment (start 13.716 13.97) (end 13.716 26.416) (width 0.38) (layer "B.Cu") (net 5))
 (segment (start -1.27 26.67) (end 0 27.94) (width 0.38) (layer "B.Cu") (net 5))
 (segment (start 13.716 11.684) (end 15.24 10.16) (width 0.38) (layer "B.Cu") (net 5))
 (segment (start 0 10.16) (end -1.27 11.43) (width 0.38) (layer "B.Cu") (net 5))
 (segment (start 12.192 28.116) (end 12.192 33.655) (width 0.38) (layer "F.Cu") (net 8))
 (segment (start 12.995 34.458) (end 12.192 33.655) (width 0.38) (layer "F.Cu") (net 8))
 (segment (start 7.366 35.3164) (end 7.6556 35.606) (width 0.38) (layer "F.Cu") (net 8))
 (segment (start 7.6556 35.606) (end 8.6406 35.606) (width 0.38) (layer "F.Cu") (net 8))
 (segment (start 13.544 38.1) (end 15.24 38.1) (width 0.38) (layer "F.Cu") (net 8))
 (segment (start 12.3444 35.6108) (end 12.3386 35.605) (width 0.38) (layer "F.Cu") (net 8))
 (segment (start 12.3386 35.605) (end 11.049 35.605) (width 0.38) (layer "F.Cu") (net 8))
 (segment (start 12.995 35.6108) (end 12.995 34.458) (width 0.38) (layer "F.Cu") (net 8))
 (segment (start 7.6856 33.706) (end 7.366 34.0256) (width 0.38) (layer "F.Cu") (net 8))
 (segment (start 12.995 37.551) (end 12.995 35.6108) (width 0.38) (layer "F.Cu") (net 8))
 (segment (start 8.6406 33.706) (end 7.6856 33.706) (width 0.38) (layer "F.Cu") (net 8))
 (segment (start 8.6406 35.606) (end 11.048 35.606) (width 0.38) (layer "F.Cu") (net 8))
 (segment (start 12.995 37.551) (end 13.544 38.1) (width 0.38) (layer "F.Cu") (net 8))
 (segment (start 7.366 34.0256) (end 7.366 35.3164) (width 0.38) (layer "F.Cu") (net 8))
 (segment (start 12.995 35.6108) (end 12.3444 35.6108) (width 0.38) (layer "F.Cu") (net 8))
 (via (at 12.192 28.116) (size 0.8) (drill 0.4) (layers "F.Cu" "B.Cu") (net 8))
 (segment (start 9.017 0) (end 12.192 3.175) (width 0.38) (layer "B.Cu") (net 8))
 (segment (start 12.192 3.175) (end 12.192 28.116) (width 0.38) (layer "B.Cu") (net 8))
 (segment (start 0 0) (end 9.017 0) (width 0.38) (layer "B.Cu") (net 8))
 (segment (start 10.685 20.809) (end 8.908997 20.809) (width 0.38) (layer "F.Cu") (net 7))
 (segment (start 6.0406 35.606) (end 6.0406 36.2608) (width 0.38) (layer "F.Cu") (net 7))
 (segment (start 3.175 36.7134) (end 2.54 36.0784) (width 0.38) (layer "F.Cu") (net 7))
 (segment (start 10.414 11.938) (end 11.193 12.717) (width 0.38) (layer "F.Cu") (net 7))
 (segment (start 6.0406 36.2608) (end 5.588 36.7134) (width 0.38) (layer "F.Cu") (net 7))
 (segment (start 3.037576 34.605) (end 3.5054 34.605) (width 0.38) (layer "F.Cu") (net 7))
 (segment (start 8.908997 20.809) (end 8.889997 20.828) (width 0.38) (layer "F.Cu") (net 7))
 (segment (start 11.193 12.717) (end 11.193 13.798) (width 0.38) (layer "F.Cu") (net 7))
 (segment (start 5.588 36.7134) (end 3.175 36.7134) (width 0.38) (layer "F.Cu") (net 7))
 (segment (start 8.808 31.451) (end 8.509 31.75) (width 0.38) (layer "F.Cu") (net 7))
 (segment (start 3.5054 34.605) (end 3.7846 34.3258) (width 0.38) (layer "F.Cu") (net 7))
 (segment (start 3.7846 34.3258) (end 3.7846 33.595) (width 0.38) (layer "F.Cu") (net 7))
 (segment (start 9.316 11.938) (end 10.414 11.938) (width 0.38) (layer "F.Cu") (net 7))
 (segment (start 2.54 35.102576) (end 3.037576 34.605) (width 0.38) (layer "F.Cu") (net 7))
 (segment (start 8.808 30.353) (end 8.808 31.451) (width 0.38) (layer "F.Cu") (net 7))
 (segment (start 9.779 13.798) (end 11.193 13.798) (width 0.38) (layer "F.Cu") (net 7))
 (segment (start 2.54 36.0784) (end 2.54 35.102576) (width 0.38) (layer "F.Cu") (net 7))
 (segment (start 8.509 31.75) (end 4.572 31.75) (width 0.38) (layer "F.Cu") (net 7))
 (segment (start 3.7846 32.5374) (end 3.7846 33.595) (width 0.38) (layer "F.Cu") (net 7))
 (segment (start 4.572 31.75) (end 3.7846 32.5374) (width 0.38) (layer "F.Cu") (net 7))
 (segment (start 8.808 29.337) (end 8.808 30.353) (width 0.38) (layer "F.Cu") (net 7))
 (via (at 8.889997 20.828) (size 0.8) (drill 0.4) (layers "F.Cu" "B.Cu") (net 7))
 (via (at 9.779 13.798) (size 0.8) (drill 0.4) (layers "F.Cu" "B.Cu") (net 7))
 (via (at 8.808 29.337) (size 0.8) (drill 0.4) (layers "F.Cu" "B.Cu") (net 7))
 (segment (start 8.808 20.909997) (end 8.808 29.337) (width 0.38) (layer "B.Cu") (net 7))
 (segment (start 9.779 13.798) (end 9.779 18.161) (width 0.38) (layer "B.Cu") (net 7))
 (segment (start 8.889997 20.828) (end 8.808 20.909997) (width 0.38) (layer "B.Cu") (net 7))
 (segment (start 9.779 18.161) (end 8.889997 19.050003) (width 0.38) (layer "B.Cu") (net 7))
 (segment (start 8.889997 19.050003) (end 8.889997 20.828) (width 0.38) (layer "B.Cu") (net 7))
 (segment (start 2.032 26.162) (end 2.835 25.359) (width 0.2) (layer "F.Cu") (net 17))
 (segment (start 2.032 28.448) (end 2.032 26.162) (width 0.2) (layer "F.Cu") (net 17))
 (segment (start 0 30.48) (end 2.032 28.448) (width 0.2) (layer "F.Cu") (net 17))
 (segment (start 2.835 25.359) (end 4.809 25.359) (width 0.2) (layer "F.Cu") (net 17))
 (segment (start 3.429 30.48) (end 3.429 26.924) (width 0.2) (layer "F.Cu") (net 19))
 (segment (start 3.694 26.659) (end 4.809 26.659) (width 0.2) (layer "F.Cu") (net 19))
 (segment (start 3.429 26.924) (end 3.694 26.659) (width 0.2) (layer "F.Cu") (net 19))
 (segment (start 1.778 33.782) (end 1.778 32.131) (width 0.2) (layer "F.Cu") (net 19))
 (segment (start 1.778 32.131) (end 3.429 30.48) (width 0.2) (layer "F.Cu") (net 19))
 (segment (start 0 35.56) (end 1.778 33.782) (width 0.2) (layer "F.Cu") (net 19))
 (segment (start 13.462 31.242) (end 13.462 27.051) (width 0.2) (layer "F.Cu") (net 22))
 (segment (start 15.24 33.02) (end 13.462 31.242) (width 0.2) (layer "F.Cu") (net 22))
 (segment (start 13.462 27.051) (end 12.42 26.009) (width 0.2) (layer "F.Cu") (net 22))
 (segment (start 12.42 26.009) (end 10.685 26.009) (width 0.2) (layer "F.Cu") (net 22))
 (segment (start 0 25.4) (end 0.691 24.709) (width 0.2) (layer "F.Cu") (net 16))
 (segment (start 0.691 24.709) (end 4.809 24.709) (width 0.2) (layer "F.Cu") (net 16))
 (segment (start 12.7 21.463) (end 12.7 17.78) (width 0.2) (layer "F.Cu") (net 28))
 (segment (start 12.7 17.78) (end 15.24 15.24) (width 0.2) (layer "F.Cu") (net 28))
 (segment (start 12.054 22.109) (end 12.7 21.463) (width 0.2) (layer "F.Cu") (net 28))
 (segment (start 10.685 22.109) (end 12.054 22.109) (width 0.2) (layer "F.Cu") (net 28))
 (segment (start 0 22.86) (end 1.199 24.059) (width 0.2) (layer "F.Cu") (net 15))
 (segment (start 1.199 24.059) (end 4.809 24.059) (width 0.2) (layer "F.Cu") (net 15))
 (segment (start 13.843 21.082) (end 13.843 19.177) (width 0.2) (layer "F.Cu") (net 27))
 (segment (start 10.685 22.759) (end 12.166 22.759) (width 0.2) (layer "F.Cu") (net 27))
 (segment (start 13.843 19.177) (end 15.24 17.78) (width 0.2) (layer "F.Cu") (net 27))
 (segment (start 12.166 22.759) (end 13.843 21.082) (width 0.2) (layer "F.Cu") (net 27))
 (segment (start 12.892 33.212) (end 15.24 35.56) (width 0.2) (layer "F.Cu") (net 21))
 (segment (start 12.892 27.37) (end 12.892 33.212) (width 0.2) (layer "F.Cu") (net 21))
 (segment (start 12.181 26.659) (end 12.892 27.37) (width 0.2) (layer "F.Cu") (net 21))
 (segment (start 10.685 26.659) (end 12.181 26.659) (width 0.2) (layer "F.Cu") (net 21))
 (segment (start 1.905 21.336) (end 1.905 20.1325) (width 0.2) (layer "F.Cu") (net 13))
 (segment (start 1.905 20.1325) (end 0 18.2275) (width 0.2) (layer "F.Cu") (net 13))
 (segment (start 4.809 22.759) (end 3.328 22.759) (width 0.2) (layer "F.Cu") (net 13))
 (segment (start 3.328 22.759) (end 1.905 21.336) (width 0.2) (layer "F.Cu") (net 13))
 (segment (start 13.97 26.416) (end 12.913 25.359) (width 0.2) (layer "F.Cu") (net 23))
 (segment (start 13.97 29.21) (end 13.97 26.416) (width 0.2) (layer "F.Cu") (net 23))
 (segment (start 15.24 30.48) (end 13.97 29.21) (width 0.2) (layer "F.Cu") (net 23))
 (segment (start 10.685 25.359) (end 12.913 25.359) (width 0.2) (layer "F.Cu") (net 23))
 (segment (start 14.041 24.059) (end 15.24 22.86) (width 0.2) (layer "F.Cu") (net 25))
 (segment (start 10.685 24.059) (end 14.041 24.059) (width 0.2) (layer "F.Cu") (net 25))
 (segment (start 2.54 21.082) (end 2.54 17.78) (width 0.2) (layer "F.Cu") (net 12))
 (segment (start 3.567 22.109) (end 2.54 21.082) (width 0.2) (layer "F.Cu") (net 12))
 (segment (start 2.54 17.78) (end 0 15.24) (width 0.2) (layer "F.Cu") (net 12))
 (segment (start 4.809 22.109) (end 3.567 22.109) (width 0.2) (layer "F.Cu") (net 12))
 (segment (start 14.549 24.709) (end 15.24 25.4) (width 0.2) (layer "F.Cu") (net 24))
 (segment (start 10.685 24.709) (end 14.549 24.709) (width 0.2) (layer "F.Cu") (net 24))
 (segment (start 10.685 23.409) (end 12.151 23.409) (width 0.2) (layer "F.Cu") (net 26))
 (segment (start 12.151 23.409) (end 15.24 20.32) (width 0.2) (layer "F.Cu") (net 26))
 (segment (start 3.089 23.409) (end 4.809 23.409) (width 0.2) (layer "F.Cu") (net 14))
 (segment (start 0 20.32) (end 3.089 23.409) (width 0.2) (layer "F.Cu") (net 14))
 (segment (start 3.201 26.009) (end 4.809 26.009) (width 0.2) (layer "F.Cu") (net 18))
 (segment (start 0 33.02) (end 2.794 30.226) (width 0.2) (layer "F.Cu") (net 18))
 (segment (start 2.794 26.416) (end 3.201 26.009) (width 0.2) (layer "F.Cu") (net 18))
 (segment (start 2.794 30.226) (end 2.794 26.416) (width 0.2) (layer "F.Cu") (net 18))
 (segment (start 10.685 27.309) (end 6.735 27.309) (width 0.2) (layer "F.Cu") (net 11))
 (segment (start 10.685 27.959) (end 10.685 27.309) (width 0.2) (layer "F.Cu") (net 11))
 (segment (start 6.735 27.309) (end 6.731 27.305) (width 0.2) (layer "F.Cu") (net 11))
 (via (at 6.731 27.305) (size 0.8) (drill 0.4) (layers "F.Cu" "B.Cu") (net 11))
 (segment (start 0 12.7) (end 2.54 15.24) (width 0.2) (layer "B.Cu") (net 11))
 (segment (start 2.54 19.685) (end 6.731 23.876) (width 0.2) (layer "B.Cu") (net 11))
 (segment (start 6.731 23.876) (end 6.731 27.305) (width 0.2) (layer "B.Cu") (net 11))
 (segment (start 2.54 15.24) (end 2.54 19.685) (width 0.2) (layer "B.Cu") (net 11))
 (segment (start 11.193 16.398) (end 9.204 16.398) (width 0.2) (layer "F.Cu") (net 1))
 (segment (start 5.317 13.798) (end 6.604 13.798) (width 0.2) (layer "F.Cu") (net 1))
 (segment (start 9.204 16.398) (end 6.604 13.798) (width 0.2) (layer "F.Cu") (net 1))
 (segment (start 4.809 20.809) (end 4.682 20.682) (width 0.2) (layer "F.Cu") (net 1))
 (segment (start 4.682 19.447998) (end 4.681998 19.447996) (width 0.2) (layer "F.Cu") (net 1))
 (segment (start 11.193 16.398) (end 11.193 17.048) (width 0.2) (layer "F.Cu") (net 1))
 (segment (start 4.682 20.682) (end 4.682 19.447998) (width 0.2) (layer "F.Cu") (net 1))
 (via (at 4.681998 19.447996) (size 0.8) (drill 0.4) (layers "F.Cu" "B.Cu") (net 1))
 (via (at 6.604 13.798) (size 0.8) (drill 0.4) (layers "F.Cu" "B.Cu") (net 1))
 (segment (start 4.681998 16.654002) (end 6.604 14.732) (width 0.2) (layer "B.Cu") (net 1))
 (segment (start 6.604 14.732) (end 6.604 13.798) (width 0.2) (layer "B.Cu") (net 1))
 (segment (start 6.604 12.573) (end 1.651 7.62) (width 0.2) (layer "B.Cu") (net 1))
 (segment (start 6.604 13.798) (end 6.604 12.573) (width 0.2) (layer "B.Cu") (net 1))
 (segment (start 1.651 7.62) (end 0 7.62) (width 0.2) (layer "B.Cu") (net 1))
 (segment (start 4.681998 19.447996) (end 4.681998 16.654002) (width 0.2) (layer "B.Cu") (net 1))
 (segment (start 4.3795 14.448) (end 5.317 14.448) (width 0.2) (layer "F.Cu") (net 2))
 (segment (start 4.2795 14.548) (end 4.3795 14.448) (width 0.2) (layer "F.Cu") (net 2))
 (segment (start 5.317 17.048) (end 4.44695 17.048) (width 0.2) (layer "F.Cu") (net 2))
 (segment (start 4.44695 17.048) (end 4.2795 16.88055) (width 0.2) (layer "F.Cu") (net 2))
 (segment (start 4.2795 16.88055) (end 4.2795 14.548) (width 0.2) (layer "F.Cu") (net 2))
 (segment (start 5.317 15.748) (end 5.317 16.398) (width 0.2) (layer "F.Cu") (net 4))
 (segment (start 9.443 17.698) (end 11.193 17.698) (width 0.2) (layer "F.Cu") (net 4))
 (segment (start 5.317 16.398) (end 8.143 16.398) (width 0.2) (layer "F.Cu") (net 4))
 (segment (start 8.143 16.398) (end 9.443 17.698) (width 0.2) (layer "F.Cu") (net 4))
 (segment (start 4.809 21.459) (end 6.854 21.459) (width 0.2) (layer "F.Cu") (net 3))
 (segment (start 6.854 21.459) (end 6.858 21.463) (width 0.2) (layer "F.Cu") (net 3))
 (segment (start 6.985 15.494) (end 6.890602 15.588398) (width 0.2) (layer "F.Cu") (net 3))
 (segment (start 6.890602 15.399602) (end 6.589 15.098) (width 0.2) (layer "F.Cu") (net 3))
 (segment (start 6.890602 15.588398) (end 6.890602 15.399602) (width 0.2) (layer "F.Cu") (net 3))
 (segment (start 6.589 15.098) (end 5.317 15.098) (width 0.2) (layer "F.Cu") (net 3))
 (via (at 6.858 21.463) (size 0.8) (drill 0.4) (layers "F.Cu" "B.Cu") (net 3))
 (via (at 6.985 15.494) (size 0.8) (drill 0.4) (layers "F.Cu" "B.Cu") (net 3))
 (segment (start 6.731 15.748) (end 6.731 20.701) (width 0.2) (layer "B.Cu") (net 3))
 (segment (start 6.731 20.701) (end 6.858 20.828) (width 0.2) (layer "B.Cu") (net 3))
 (segment (start 6.985 15.494) (end 6.731 15.748) (width 0.2) (layer "B.Cu") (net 3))
 (segment (start 6.858 20.828) (end 6.858 21.463) (width 0.2) (layer "B.Cu") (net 3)))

